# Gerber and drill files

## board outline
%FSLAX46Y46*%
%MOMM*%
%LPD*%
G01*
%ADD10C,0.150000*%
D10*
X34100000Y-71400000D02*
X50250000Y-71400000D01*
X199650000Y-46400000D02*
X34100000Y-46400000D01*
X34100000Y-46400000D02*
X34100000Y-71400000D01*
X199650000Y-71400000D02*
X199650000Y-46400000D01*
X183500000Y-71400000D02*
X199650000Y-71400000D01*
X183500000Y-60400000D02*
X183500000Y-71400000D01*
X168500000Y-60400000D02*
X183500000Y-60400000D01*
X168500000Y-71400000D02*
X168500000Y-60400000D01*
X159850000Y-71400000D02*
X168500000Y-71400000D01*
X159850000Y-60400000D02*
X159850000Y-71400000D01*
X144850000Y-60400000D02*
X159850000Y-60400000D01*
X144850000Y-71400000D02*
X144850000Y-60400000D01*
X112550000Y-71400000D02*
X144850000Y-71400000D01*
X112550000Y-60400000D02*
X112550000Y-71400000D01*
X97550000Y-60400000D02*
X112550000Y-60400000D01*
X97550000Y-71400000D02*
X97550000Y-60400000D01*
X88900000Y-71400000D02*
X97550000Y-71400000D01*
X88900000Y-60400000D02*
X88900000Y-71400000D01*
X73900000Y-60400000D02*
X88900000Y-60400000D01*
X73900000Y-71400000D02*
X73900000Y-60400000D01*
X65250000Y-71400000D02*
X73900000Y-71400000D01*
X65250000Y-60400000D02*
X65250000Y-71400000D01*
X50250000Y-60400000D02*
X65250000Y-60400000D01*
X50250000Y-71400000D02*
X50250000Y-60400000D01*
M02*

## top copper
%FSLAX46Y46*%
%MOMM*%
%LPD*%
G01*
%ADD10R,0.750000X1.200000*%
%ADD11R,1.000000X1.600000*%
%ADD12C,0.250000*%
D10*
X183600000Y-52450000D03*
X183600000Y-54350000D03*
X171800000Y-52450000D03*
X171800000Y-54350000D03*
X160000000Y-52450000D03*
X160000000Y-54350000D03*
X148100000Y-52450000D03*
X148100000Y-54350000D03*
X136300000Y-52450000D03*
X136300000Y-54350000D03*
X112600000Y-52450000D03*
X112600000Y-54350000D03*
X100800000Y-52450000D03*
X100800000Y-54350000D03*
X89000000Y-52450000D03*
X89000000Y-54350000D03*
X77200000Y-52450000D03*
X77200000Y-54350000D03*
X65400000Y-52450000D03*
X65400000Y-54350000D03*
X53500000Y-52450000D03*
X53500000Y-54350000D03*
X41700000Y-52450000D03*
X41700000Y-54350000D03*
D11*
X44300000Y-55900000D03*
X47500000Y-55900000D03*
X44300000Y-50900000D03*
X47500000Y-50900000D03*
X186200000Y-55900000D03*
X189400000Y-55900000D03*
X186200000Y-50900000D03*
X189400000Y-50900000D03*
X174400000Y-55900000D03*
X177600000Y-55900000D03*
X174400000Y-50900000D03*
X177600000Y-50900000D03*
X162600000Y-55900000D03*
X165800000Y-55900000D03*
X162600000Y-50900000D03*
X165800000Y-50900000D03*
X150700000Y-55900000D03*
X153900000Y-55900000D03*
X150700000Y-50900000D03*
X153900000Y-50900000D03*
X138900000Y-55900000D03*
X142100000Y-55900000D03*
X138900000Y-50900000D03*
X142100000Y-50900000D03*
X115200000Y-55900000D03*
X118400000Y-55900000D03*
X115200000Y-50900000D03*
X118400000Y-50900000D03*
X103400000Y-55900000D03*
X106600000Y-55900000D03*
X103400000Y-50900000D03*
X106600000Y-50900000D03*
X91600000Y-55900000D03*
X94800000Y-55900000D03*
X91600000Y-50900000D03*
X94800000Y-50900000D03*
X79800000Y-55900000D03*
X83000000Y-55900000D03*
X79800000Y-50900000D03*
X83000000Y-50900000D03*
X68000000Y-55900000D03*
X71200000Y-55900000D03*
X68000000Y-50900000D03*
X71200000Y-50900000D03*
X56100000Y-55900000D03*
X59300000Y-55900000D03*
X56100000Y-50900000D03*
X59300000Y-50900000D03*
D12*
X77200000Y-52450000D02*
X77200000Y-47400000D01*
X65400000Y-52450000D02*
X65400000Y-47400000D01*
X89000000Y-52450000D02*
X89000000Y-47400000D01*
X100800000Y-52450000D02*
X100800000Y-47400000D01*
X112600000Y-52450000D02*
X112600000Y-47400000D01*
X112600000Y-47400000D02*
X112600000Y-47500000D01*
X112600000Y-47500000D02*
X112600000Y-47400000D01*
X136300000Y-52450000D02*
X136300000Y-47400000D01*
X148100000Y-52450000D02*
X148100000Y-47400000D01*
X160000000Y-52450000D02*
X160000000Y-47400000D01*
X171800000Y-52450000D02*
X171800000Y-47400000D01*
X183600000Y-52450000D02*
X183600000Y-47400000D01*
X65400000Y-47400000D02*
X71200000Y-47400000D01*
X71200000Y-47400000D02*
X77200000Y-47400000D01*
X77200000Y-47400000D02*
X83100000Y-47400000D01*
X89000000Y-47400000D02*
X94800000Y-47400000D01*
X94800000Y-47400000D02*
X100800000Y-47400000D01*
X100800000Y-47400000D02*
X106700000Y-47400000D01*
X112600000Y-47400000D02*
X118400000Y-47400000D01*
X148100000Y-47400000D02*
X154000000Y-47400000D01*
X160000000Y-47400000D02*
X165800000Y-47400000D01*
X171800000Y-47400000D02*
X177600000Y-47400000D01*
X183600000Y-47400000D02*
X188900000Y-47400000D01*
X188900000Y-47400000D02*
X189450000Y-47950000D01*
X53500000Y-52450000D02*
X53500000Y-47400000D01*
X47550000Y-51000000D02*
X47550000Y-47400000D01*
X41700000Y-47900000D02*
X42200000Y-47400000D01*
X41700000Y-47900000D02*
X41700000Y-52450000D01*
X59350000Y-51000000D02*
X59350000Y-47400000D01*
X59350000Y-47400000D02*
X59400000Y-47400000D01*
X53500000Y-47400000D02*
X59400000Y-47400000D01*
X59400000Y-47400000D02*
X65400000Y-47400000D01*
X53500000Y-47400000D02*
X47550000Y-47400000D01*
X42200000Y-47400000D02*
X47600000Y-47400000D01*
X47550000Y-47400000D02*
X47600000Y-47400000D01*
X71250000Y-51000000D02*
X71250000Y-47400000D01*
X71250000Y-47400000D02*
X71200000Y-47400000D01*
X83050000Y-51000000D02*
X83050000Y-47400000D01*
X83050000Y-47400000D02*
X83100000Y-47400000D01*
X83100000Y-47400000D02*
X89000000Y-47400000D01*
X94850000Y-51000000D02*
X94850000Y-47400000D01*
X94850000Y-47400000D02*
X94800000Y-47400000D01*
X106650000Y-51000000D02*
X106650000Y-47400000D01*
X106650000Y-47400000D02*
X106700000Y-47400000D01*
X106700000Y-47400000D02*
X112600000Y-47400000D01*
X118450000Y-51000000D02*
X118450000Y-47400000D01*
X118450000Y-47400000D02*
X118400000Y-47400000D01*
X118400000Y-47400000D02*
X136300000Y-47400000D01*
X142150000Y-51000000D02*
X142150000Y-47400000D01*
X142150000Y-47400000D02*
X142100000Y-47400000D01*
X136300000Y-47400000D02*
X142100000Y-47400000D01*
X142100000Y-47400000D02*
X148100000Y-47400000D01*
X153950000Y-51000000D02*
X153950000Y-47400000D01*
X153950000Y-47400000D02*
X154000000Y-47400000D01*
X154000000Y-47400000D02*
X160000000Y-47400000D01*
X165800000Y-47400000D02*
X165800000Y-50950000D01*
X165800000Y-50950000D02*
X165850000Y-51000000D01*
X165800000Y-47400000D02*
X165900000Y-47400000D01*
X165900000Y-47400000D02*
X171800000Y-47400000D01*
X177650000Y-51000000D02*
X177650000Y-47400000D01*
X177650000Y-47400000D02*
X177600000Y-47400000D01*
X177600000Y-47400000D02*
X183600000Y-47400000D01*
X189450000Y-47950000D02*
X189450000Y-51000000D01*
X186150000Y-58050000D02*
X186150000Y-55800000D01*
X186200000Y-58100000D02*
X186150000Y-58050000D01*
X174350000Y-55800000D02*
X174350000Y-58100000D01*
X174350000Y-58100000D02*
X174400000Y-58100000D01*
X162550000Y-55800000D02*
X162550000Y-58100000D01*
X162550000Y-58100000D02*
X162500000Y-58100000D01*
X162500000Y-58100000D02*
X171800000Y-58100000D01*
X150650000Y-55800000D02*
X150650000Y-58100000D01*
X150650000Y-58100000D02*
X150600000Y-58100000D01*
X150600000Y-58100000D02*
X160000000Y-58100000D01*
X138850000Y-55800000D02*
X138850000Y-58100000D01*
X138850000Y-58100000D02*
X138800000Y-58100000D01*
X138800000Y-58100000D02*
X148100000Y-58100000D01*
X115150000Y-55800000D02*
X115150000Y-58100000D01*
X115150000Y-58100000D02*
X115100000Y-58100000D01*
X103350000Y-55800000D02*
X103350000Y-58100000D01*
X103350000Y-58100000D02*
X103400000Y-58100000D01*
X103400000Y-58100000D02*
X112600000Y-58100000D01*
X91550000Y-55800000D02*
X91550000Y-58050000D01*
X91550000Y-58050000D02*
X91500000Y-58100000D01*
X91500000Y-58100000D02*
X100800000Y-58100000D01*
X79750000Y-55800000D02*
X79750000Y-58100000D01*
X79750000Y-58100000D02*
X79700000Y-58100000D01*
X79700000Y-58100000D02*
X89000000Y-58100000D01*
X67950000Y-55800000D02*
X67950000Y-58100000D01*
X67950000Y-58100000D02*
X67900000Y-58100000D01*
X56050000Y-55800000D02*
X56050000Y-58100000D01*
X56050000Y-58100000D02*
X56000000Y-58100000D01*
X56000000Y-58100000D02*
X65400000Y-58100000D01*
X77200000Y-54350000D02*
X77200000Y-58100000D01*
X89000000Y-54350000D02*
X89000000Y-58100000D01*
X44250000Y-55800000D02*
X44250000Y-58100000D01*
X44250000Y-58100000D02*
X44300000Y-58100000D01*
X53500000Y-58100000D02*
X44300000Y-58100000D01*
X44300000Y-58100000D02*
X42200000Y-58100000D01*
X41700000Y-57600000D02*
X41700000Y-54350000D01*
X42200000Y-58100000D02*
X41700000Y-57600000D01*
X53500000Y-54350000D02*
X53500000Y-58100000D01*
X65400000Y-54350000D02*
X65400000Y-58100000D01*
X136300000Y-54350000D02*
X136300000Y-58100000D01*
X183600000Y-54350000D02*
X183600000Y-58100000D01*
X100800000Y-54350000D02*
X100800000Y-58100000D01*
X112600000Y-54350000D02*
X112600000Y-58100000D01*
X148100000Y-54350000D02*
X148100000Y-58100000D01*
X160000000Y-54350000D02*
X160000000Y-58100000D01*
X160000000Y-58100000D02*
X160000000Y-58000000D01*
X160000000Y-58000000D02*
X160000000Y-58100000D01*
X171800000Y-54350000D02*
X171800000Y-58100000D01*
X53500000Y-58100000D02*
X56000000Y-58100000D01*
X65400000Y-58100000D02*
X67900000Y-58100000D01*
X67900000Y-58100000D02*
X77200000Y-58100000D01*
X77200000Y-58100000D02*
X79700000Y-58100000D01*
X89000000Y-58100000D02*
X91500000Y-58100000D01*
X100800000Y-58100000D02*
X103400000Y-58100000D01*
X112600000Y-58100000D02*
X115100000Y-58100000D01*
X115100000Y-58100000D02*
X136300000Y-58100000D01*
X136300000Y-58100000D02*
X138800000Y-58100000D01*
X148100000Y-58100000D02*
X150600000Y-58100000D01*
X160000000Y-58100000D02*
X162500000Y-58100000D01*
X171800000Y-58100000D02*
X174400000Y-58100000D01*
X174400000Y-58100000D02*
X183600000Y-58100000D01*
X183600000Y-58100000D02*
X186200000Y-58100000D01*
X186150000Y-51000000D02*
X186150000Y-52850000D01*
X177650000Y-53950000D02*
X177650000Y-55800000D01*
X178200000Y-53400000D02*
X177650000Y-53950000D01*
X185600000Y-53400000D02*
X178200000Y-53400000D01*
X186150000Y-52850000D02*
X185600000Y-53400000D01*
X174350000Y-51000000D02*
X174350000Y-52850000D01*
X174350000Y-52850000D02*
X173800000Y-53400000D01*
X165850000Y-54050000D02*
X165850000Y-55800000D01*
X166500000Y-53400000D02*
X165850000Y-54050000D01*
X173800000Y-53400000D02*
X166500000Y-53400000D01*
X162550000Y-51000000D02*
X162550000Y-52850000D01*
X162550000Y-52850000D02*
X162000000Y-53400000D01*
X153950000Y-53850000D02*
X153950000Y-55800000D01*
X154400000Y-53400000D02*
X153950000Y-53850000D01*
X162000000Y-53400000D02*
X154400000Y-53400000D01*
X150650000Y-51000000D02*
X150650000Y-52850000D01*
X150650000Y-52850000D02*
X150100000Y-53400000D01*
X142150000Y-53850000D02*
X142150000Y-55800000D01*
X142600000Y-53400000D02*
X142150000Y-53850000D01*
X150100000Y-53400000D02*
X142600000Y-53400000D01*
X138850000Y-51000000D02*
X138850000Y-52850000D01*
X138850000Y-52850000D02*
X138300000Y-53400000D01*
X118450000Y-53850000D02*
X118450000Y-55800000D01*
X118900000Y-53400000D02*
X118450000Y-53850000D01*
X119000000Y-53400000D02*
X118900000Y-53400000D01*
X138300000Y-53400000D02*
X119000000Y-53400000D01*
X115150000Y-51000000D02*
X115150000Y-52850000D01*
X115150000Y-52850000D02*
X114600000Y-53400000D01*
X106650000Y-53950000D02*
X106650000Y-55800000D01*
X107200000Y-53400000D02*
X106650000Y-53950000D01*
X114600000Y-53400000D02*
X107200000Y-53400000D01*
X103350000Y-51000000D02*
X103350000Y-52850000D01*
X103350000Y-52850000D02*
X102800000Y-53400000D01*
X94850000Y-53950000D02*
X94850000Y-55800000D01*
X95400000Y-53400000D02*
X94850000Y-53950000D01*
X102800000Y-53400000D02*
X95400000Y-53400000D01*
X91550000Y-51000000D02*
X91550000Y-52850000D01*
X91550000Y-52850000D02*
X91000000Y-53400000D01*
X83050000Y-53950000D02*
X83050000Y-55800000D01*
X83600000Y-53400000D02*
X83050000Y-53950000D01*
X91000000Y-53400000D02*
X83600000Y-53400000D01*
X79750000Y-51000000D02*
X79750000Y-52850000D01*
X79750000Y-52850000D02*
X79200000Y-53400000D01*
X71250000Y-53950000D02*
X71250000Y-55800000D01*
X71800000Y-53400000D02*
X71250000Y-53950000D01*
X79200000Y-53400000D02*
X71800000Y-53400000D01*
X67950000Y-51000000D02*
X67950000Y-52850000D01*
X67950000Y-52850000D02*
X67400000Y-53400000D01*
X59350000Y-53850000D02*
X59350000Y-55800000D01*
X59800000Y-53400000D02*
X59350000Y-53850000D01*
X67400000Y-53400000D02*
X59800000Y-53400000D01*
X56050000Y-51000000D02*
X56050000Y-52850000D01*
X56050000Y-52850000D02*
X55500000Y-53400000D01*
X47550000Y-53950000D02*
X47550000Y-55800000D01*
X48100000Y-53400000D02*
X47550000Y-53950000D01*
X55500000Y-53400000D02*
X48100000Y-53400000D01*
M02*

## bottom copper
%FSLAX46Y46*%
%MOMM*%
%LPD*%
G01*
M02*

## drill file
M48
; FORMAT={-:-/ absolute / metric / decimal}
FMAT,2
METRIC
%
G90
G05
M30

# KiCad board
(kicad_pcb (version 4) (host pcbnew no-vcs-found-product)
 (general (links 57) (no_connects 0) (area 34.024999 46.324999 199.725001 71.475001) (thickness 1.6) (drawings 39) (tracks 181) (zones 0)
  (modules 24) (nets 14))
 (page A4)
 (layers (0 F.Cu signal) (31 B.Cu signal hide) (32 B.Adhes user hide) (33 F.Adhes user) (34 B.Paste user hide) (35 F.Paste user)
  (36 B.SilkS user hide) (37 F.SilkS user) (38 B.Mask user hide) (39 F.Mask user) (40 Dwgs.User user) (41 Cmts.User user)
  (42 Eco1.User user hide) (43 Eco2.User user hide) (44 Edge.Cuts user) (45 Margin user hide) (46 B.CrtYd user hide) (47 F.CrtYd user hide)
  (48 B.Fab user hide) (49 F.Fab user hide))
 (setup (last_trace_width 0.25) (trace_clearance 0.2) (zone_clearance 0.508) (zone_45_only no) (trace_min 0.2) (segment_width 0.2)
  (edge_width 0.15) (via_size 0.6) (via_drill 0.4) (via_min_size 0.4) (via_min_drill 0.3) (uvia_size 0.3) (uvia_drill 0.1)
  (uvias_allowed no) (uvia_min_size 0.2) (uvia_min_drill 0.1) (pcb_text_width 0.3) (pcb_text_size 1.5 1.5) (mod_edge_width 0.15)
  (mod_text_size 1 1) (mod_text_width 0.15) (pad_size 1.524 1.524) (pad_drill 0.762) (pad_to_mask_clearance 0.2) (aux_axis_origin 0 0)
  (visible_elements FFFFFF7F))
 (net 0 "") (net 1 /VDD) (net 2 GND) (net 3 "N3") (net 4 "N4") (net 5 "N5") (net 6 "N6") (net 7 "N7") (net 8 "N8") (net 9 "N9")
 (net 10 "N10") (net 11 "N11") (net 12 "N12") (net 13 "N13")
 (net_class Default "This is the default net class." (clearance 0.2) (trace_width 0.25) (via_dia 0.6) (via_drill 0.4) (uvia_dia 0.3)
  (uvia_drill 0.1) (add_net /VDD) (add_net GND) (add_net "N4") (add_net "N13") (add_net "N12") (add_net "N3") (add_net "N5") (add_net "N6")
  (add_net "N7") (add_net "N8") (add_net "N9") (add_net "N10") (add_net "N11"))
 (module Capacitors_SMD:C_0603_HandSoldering (layer F.Cu) (at 183.6 53.4 270)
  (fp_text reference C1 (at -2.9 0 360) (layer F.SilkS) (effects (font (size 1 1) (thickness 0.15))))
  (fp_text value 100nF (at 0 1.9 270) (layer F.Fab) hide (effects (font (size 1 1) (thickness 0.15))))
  (pad 1 smd rect (at -0.95 0 270) (size 1.2 0.75) (layers F.Cu F.Paste F.Mask) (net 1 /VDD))
  (pad 2 smd rect (at 0.95 0 270) (size 1.2 0.75) (layers F.Cu F.Paste F.Mask) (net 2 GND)))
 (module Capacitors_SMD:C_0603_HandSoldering (layer F.Cu) (at 171.8 53.4 270)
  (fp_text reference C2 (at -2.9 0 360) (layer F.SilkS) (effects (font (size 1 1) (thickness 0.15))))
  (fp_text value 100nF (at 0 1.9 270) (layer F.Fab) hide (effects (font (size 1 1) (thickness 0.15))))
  (pad 1 smd rect (at -0.95 0 270) (size 1.2 0.75) (layers F.Cu F.Paste F.Mask) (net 1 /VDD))
  (pad 2 smd rect (at 0.95 0 270) (size 1.2 0.75) (layers F.Cu F.Paste F.Mask) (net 2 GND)))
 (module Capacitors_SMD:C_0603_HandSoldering (layer F.Cu) (at 160 53.4 270)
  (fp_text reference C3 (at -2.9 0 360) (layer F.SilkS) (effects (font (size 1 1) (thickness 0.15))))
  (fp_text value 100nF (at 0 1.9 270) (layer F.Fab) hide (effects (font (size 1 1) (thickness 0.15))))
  (pad 1 smd rect (at -0.95 0 270) (size 1.2 0.75) (layers F.Cu F.Paste F.Mask) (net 1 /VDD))
  (pad 2 smd rect (at 0.95 0 270) (size 1.2 0.75) (layers F.Cu F.Paste F.Mask) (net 2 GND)))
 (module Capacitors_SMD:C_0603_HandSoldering (layer F.Cu) (at 148.1 53.4 270)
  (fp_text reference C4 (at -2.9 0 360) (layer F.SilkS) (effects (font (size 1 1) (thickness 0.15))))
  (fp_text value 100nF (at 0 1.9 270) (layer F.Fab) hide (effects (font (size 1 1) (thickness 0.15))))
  (pad 1 smd rect (at -0.95 0 270) (size 1.2 0.75) (layers F.Cu F.Paste F.Mask) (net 1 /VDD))
  (pad 2 smd rect (at 0.95 0 270) (size 1.2 0.75) (layers F.Cu F.Paste F.Mask) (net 2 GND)))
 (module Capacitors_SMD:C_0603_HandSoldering (layer F.Cu) (at 136.3 53.4 270)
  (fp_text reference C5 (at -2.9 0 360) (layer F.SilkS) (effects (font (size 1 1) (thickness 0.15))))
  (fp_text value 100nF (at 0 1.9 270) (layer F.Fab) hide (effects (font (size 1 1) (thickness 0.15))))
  (pad 1 smd rect (at -0.95 0 270) (size 1.2 0.75) (layers F.Cu F.Paste F.Mask) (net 1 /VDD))
  (pad 2 smd rect (at 0.95 0 270) (size 1.2 0.75) (layers F.Cu F.Paste F.Mask) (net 2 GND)))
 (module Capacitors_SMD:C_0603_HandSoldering (layer F.Cu) (at 112.6 53.4 270)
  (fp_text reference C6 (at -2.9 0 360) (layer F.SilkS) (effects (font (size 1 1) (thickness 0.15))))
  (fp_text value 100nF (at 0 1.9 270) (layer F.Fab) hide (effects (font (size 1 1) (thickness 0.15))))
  (pad 1 smd rect (at -0.95 0 270) (size 1.2 0.75) (layers F.Cu F.Paste F.Mask) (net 1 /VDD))
  (pad 2 smd rect (at 0.95 0 270) (size 1.2 0.75) (layers F.Cu F.Paste F.Mask) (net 2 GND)))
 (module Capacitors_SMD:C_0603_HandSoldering (layer F.Cu) (at 100.8 53.4 270)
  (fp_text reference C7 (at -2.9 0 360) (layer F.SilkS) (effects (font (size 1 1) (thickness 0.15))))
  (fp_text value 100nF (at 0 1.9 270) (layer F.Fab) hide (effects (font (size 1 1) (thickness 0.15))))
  (pad 1 smd rect (at -0.95 0 270) (size 1.2 0.75) (layers F.Cu F.Paste F.Mask) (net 1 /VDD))
  (pad 2 smd rect (at 0.95 0 270) (size 1.2 0.75) (layers F.Cu F.Paste F.Mask) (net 2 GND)))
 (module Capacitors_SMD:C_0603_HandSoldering (layer F.Cu) (at 89 53.4 270)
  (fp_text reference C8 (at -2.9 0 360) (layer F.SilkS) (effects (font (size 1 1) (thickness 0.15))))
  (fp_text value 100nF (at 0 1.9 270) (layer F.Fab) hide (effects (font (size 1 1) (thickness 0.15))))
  (pad 1 smd rect (at -0.95 0 270) (size 1.2 0.75) (layers F.Cu F.Paste F.Mask) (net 1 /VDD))
  (pad 2 smd rect (at 0.95 0 270) (size 1.2 0.75) (layers F.Cu F.Paste F.Mask) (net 2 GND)))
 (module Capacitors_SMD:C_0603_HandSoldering (layer F.Cu) (at 77.2 53.4 270)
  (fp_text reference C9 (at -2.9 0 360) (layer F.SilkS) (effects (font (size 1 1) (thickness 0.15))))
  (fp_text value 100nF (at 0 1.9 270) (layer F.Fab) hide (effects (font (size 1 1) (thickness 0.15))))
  (pad 1 smd rect (at -0.95 0 270) (size 1.2 0.75) (layers F.Cu F.Paste F.Mask) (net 1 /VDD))
  (pad 2 smd rect (at 0.95 0 270) (size 1.2 0.75) (layers F.Cu F.Paste F.Mask) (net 2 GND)))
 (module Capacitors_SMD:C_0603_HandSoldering (layer F.Cu) (at 65.4 53.4 270)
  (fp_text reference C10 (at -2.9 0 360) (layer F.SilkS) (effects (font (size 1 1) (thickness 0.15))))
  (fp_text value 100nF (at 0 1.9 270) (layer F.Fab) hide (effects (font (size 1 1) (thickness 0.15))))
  (pad 1 smd rect (at -0.95 0 270) (size 1.2 0.75) (layers F.Cu F.Paste F.Mask) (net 1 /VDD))
  (pad 2 smd rect (at 0.95 0 270) (size 1.2 0.75) (layers F.Cu F.Paste F.Mask) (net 2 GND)))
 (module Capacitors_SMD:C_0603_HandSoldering (layer F.Cu) (at 53.5 53.4 270)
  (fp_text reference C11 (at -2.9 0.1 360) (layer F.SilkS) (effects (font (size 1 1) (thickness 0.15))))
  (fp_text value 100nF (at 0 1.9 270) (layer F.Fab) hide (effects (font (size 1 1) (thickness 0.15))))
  (pad 1 smd rect (at -0.95 0 270) (size 1.2 0.75) (layers F.Cu F.Paste F.Mask) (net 1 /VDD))
  (pad 2 smd rect (at 0.95 0 270) (size 1.2 0.75) (layers F.Cu F.Paste F.Mask) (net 2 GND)))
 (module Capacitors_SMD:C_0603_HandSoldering (layer F.Cu) (at 41.7 53.4 270)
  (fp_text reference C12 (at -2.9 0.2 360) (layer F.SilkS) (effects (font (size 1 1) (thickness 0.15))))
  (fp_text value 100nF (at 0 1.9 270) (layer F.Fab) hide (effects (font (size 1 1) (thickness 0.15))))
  (pad 1 smd rect (at -0.95 0 270) (size 1.2 0.75) (layers F.Cu F.Paste F.Mask) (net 1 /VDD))
  (pad 2 smd rect (at 0.95 0 270) (size 1.2 0.75) (layers F.Cu F.Paste F.Mask) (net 2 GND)))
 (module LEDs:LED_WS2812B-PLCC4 (layer F.Cu) (at 45.9 53.4 270)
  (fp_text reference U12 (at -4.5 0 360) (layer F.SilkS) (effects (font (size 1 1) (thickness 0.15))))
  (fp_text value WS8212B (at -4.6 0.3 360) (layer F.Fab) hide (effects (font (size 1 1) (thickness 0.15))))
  (pad 3 smd rect (at 2.5 1.6 270) (size 1.6 1) (layers F.Cu F.Paste F.Mask) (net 2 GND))
  (pad 4 smd rect (at 2.5 -1.6 270) (size 1.6 1) (layers F.Cu F.Paste F.Mask) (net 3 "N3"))
  (pad 2 smd rect (at -2.5 1.6 270) (size 1.6 1) (layers F.Cu F.Paste F.Mask))
  (pad 1 smd rect (at -2.5 -1.6 270) (size 1.6 1) (layers F.Cu F.Paste F.Mask) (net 1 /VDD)))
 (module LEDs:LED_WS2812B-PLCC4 (layer F.Cu) (at 187.8 53.4 270)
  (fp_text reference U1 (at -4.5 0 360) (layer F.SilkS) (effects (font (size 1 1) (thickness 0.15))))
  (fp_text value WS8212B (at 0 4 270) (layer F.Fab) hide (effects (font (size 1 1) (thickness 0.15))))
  (pad 3 smd rect (at 2.5 1.6 270) (size 1.6 1) (layers F.Cu F.Paste F.Mask) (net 2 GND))
  (pad 4 smd rect (at 2.5 -1.6 270) (size 1.6 1) (layers F.Cu F.Paste F.Mask))
  (pad 2 smd rect (at -2.5 1.6 270) (size 1.6 1) (layers F.Cu F.Paste F.Mask) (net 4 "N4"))
  (pad 1 smd rect (at -2.5 -1.6 270) (size 1.6 1) (layers F.Cu F.Paste F.Mask) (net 1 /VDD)))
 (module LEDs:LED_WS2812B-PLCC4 (layer F.Cu) (at 176 53.4 270)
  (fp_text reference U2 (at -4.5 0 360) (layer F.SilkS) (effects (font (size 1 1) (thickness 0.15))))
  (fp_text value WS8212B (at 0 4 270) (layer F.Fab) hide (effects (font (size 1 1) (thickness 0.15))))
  (pad 3 smd rect (at 2.5 1.6 270) (size 1.6 1) (layers F.Cu F.Paste F.Mask) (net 2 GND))
  (pad 4 smd rect (at 2.5 -1.6 270) (size 1.6 1) (layers F.Cu F.Paste F.Mask) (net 4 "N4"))
  (pad 2 smd rect (at -2.5 1.6 270) (size 1.6 1) (layers F.Cu F.Paste F.Mask) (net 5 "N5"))
  (pad 1 smd rect (at -2.5 -1.6 270) (size 1.6 1) (layers F.Cu F.Paste F.Mask) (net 1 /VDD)))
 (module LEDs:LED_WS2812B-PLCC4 (layer F.Cu) (at 164.2 53.4 270)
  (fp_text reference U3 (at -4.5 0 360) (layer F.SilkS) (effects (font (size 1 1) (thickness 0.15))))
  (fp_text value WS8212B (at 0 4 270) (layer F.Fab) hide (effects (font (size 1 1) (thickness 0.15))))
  (pad 3 smd rect (at 2.5 1.6 270) (size 1.6 1) (layers F.Cu F.Paste F.Mask) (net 2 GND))
  (pad 4 smd rect (at 2.5 -1.6 270) (size 1.6 1) (layers F.Cu F.Paste F.Mask) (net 5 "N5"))
  (pad 2 smd rect (at -2.5 1.6 270) (size 1.6 1) (layers F.Cu F.Paste F.Mask) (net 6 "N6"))
  (pad 1 smd rect (at -2.5 -1.6 270) (size 1.6 1) (layers F.Cu F.Paste F.Mask) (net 1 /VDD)))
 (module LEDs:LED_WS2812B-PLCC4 (layer F.Cu) (at 152.3 53.4 270)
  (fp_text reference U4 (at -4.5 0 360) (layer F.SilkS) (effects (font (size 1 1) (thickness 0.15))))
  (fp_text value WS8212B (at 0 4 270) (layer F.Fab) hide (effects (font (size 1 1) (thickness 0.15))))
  (pad 3 smd rect (at 2.5 1.6 270) (size 1.6 1) (layers F.Cu F.Paste F.Mask) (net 2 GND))
  (pad 4 smd rect (at 2.5 -1.6 270) (size 1.6 1) (layers F.Cu F.Paste F.Mask) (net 6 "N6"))
  (pad 2 smd rect (at -2.5 1.6 270) (size 1.6 1) (layers F.Cu F.Paste F.Mask) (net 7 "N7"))
  (pad 1 smd rect (at -2.5 -1.6 270) (size 1.6 1) (layers F.Cu F.Paste F.Mask) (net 1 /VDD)))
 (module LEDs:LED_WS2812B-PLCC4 (layer F.Cu) (at 140.5 53.4 270)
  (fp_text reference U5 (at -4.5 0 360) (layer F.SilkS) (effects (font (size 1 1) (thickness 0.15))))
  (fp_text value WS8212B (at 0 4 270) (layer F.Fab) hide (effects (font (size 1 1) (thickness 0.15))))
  (pad 3 smd rect (at 2.5 1.6 270) (size 1.6 1) (layers F.Cu F.Paste F.Mask) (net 2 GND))
  (pad 4 smd rect (at 2.5 -1.6 270) (size 1.6 1) (layers F.Cu F.Paste F.Mask) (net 7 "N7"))
  (pad 2 smd rect (at -2.5 1.6 270) (size 1.6 1) (layers F.Cu F.Paste F.Mask) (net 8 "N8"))
  (pad 1 smd rect (at -2.5 -1.6 270) (size 1.6 1) (layers F.Cu F.Paste F.Mask) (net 1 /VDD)))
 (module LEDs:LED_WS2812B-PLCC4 (layer F.Cu) (at 116.8 53.4 270)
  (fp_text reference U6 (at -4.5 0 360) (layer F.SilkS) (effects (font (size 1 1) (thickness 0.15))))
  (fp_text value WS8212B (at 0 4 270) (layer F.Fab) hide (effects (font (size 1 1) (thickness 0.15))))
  (pad 3 smd rect (at 2.5 1.6 270) (size 1.6 1) (layers F.Cu F.Paste F.Mask) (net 2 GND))
  (pad 4 smd rect (at 2.5 -1.6 270) (size 1.6 1) (layers F.Cu F.Paste F.Mask) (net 8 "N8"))
  (pad 2 smd rect (at -2.5 1.6 270) (size 1.6 1) (layers F.Cu F.Paste F.Mask) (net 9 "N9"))
  (pad 1 smd rect (at -2.5 -1.6 270) (size 1.6 1) (layers F.Cu F.Paste F.Mask) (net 1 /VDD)))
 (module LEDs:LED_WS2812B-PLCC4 (layer F.Cu) (at 105 53.4 270)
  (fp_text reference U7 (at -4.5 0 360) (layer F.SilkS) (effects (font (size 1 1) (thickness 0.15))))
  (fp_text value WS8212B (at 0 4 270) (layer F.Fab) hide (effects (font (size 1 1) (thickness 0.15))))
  (pad 3 smd rect (at 2.5 1.6 270) (size 1.6 1) (layers F.Cu F.Paste F.Mask) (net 2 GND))
  (pad 4 smd rect (at 2.5 -1.6 270) (size 1.6 1) (layers F.Cu F.Paste F.Mask) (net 9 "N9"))
  (pad 2 smd rect (at -2.5 1.6 270) (size 1.6 1) (layers F.Cu F.Paste F.Mask) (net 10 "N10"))
  (pad 1 smd rect (at -2.5 -1.6 270) (size 1.6 1) (layers F.Cu F.Paste F.Mask) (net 1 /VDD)))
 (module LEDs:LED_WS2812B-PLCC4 (layer F.Cu) (at 93.2 53.4 270)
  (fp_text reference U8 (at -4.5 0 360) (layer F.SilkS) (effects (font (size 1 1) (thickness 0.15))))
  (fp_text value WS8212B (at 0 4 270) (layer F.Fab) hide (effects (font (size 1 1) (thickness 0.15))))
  (pad 3 smd rect (at 2.5 1.6 270) (size 1.6 1) (layers F.Cu F.Paste F.Mask) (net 2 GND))
  (pad 4 smd rect (at 2.5 -1.6 270) (size 1.6 1) (layers F.Cu F.Paste F.Mask) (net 10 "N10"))
  (pad 2 smd rect (at -2.5 1.6 270) (size 1.6 1) (layers F.Cu F.Paste F.Mask) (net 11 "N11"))
  (pad 1 smd rect (at -2.5 -1.6 270) (size 1.6 1) (layers F.Cu F.Paste F.Mask) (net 1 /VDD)))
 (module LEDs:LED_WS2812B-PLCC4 (layer F.Cu) (at 81.4 53.4 270)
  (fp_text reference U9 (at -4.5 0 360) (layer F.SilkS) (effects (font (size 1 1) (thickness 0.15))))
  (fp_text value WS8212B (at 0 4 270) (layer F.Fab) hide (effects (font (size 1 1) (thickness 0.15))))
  (pad 3 smd rect (at 2.5 1.6 270) (size 1.6 1) (layers F.Cu F.Paste F.Mask) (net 2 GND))
  (pad 4 smd rect (at 2.5 -1.6 270) (size 1.6 1) (layers F.Cu F.Paste F.Mask) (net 11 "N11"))
  (pad 2 smd rect (at -2.5 1.6 270) (size 1.6 1) (layers F.Cu F.Paste F.Mask) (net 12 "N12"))
  (pad 1 smd rect (at -2.5 -1.6 270) (size 1.6 1) (layers F.Cu F.Paste F.Mask) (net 1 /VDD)))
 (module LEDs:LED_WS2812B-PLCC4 (layer F.Cu) (at 69.6 53.4 270)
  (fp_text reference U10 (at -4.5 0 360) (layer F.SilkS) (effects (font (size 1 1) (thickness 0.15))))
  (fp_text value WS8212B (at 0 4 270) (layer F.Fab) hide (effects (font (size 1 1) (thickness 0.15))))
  (pad 3 smd rect (at 2.5 1.6 270) (size 1.6 1) (layers F.Cu F.Paste F.Mask) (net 2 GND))
  (pad 4 smd rect (at 2.5 -1.6 270) (size 1.6 1) (layers F.Cu F.Paste F.Mask) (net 12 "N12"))
  (pad 2 smd rect (at -2.5 1.6 270) (size 1.6 1) (layers F.Cu F.Paste F.Mask) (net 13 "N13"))
  (pad 1 smd rect (at -2.5 -1.6 270) (size 1.6 1) (layers F.Cu F.Paste F.Mask) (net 1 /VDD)))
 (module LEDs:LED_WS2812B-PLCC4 (layer F.Cu) (at 57.7 53.4 270)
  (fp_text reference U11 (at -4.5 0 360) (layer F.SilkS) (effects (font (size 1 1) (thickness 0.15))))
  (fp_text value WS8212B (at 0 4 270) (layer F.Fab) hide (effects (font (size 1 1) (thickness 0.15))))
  (pad 3 smd rect (at 2.5 1.6 270) (size 1.6 1) (layers F.Cu F.Paste F.Mask) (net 2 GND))
  (pad 4 smd rect (at 2.5 -1.6 270) (size 1.6 1) (layers F.Cu F.Paste F.Mask) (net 13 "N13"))
  (pad 2 smd rect (at -2.5 1.6 270) (size 1.6 1) (layers F.Cu F.Paste F.Mask) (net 3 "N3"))
  (pad 1 smd rect (at -2.5 -1.6 270) (size 1.6 1) (layers F.Cu F.Paste F.Mask) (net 1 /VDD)))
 (gr_line (start 34.1 71.4) (end 50.25 71.4) (angle 90) (layer Edge.Cuts) (width 0.15))
 (gr_line (start 199.65 46.4) (end 34.1 46.4) (angle 90) (layer Edge.Cuts) (width 0.15))
 (gr_line (start 34.1 46.4) (end 34.1 71.4) (angle 90) (layer Edge.Cuts) (width 0.15))
 (gr_line (start 199.65 71.4) (end 199.65 46.4) (angle 90) (layer Edge.Cuts) (width 0.15))
 (gr_line (start 183.5 71.4) (end 199.65 71.4) (angle 90) (layer Edge.Cuts) (width 0.15))
 (gr_line (start 183.5 60.4) (end 183.5 71.4) (angle 90) (layer Edge.Cuts) (width 0.15))
 (gr_line (start 168.5 60.4) (end 183.5 60.4) (angle 90) (layer Edge.Cuts) (width 0.15))
 (gr_line (start 168.5 71.4) (end 168.5 60.4) (angle 90) (layer Edge.Cuts) (width 0.15))
 (gr_line (start 159.85 71.4) (end 168.5 71.4) (angle 90) (layer Edge.Cuts) (width 0.15))
 (gr_line (start 159.85 60.4) (end 159.85 71.4) (angle 90) (layer Edge.Cuts) (width 0.15))
 (gr_line (start 144.85 60.4) (end 159.85 60.4) (angle 90) (layer Edge.Cuts) (width 0.15))
 (gr_line (start 144.85 71.4) (end 144.85 60.4) (angle 90) (layer Edge.Cuts) (width 0.15))
 (gr_line (start 112.55 71.4) (end 144.85 71.4) (angle 90) (layer Edge.Cuts) (width 0.15))
 (gr_line (start 112.55 60.4) (end 112.55 71.4) (angle 90) (layer Edge.Cuts) (width 0.15))
 (gr_line (start 97.55 60.4) (end 112.55 60.4) (angle 90) (layer Edge.Cuts) (width 0.15))
 (gr_line (start 97.55 71.4) (end 97.55 60.4) (angle 90) (layer Edge.Cuts) (width 0.15))
 (gr_line (start 88.9 71.4) (end 97.55 71.4) (angle 90) (layer Edge.Cuts) (width 0.15))
 (gr_line (start 88.9 60.4) (end 88.9 71.4) (angle 90) (layer Edge.Cuts) (width 0.15))
 (gr_line (start 73.9 60.4) (end 88.9 60.4) (angle 90) (layer Edge.Cuts) (width 0.15))
 (gr_line (start 73.9 71.4) (end 73.9 60.4) (angle 90) (layer Edge.Cuts) (width 0.15))
 (gr_line (start 65.25 71.4) (end 73.9 71.4) (angle 90) (layer Edge.Cuts) (width 0.15))
 (gr_line (start 65.25 60.4) (end 65.25 71.4) (angle 90) (layer Edge.Cuts) (width 0.15))
 (gr_line (start 50.25 60.4) (end 65.25 60.4) (angle 90) (layer Edge.Cuts) (width 0.15))
 (gr_line (start 50.25 71.4) (end 50.25 60.4) (angle 90) (layer Edge.Cuts) (width 0.15))
 (segment (start 77.2 52.45) (end 77.2 47.4) (width 0.25) (layer F.Cu) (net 1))
 (segment (start 65.4 52.45) (end 65.4 47.4) (width 0.25) (layer F.Cu) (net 1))
 (segment (start 89 52.45) (end 89 47.4) (width 0.25) (layer F.Cu) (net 1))
 (segment (start 100.8 52.45) (end 100.8 47.4) (width 0.25) (layer F.Cu) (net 1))
 (segment (start 112.6 52.45) (end 112.6 47.4) (width 0.25) (layer F.Cu) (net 1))
 (segment (start 112.6 47.4) (end 112.6 47.5) (width 0.25) (layer F.Cu) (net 1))
 (segment (start 112.6 47.5) (end 112.6 47.4) (width 0.25) (layer F.Cu) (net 1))
 (segment (start 136.3 52.45) (end 136.3 47.4) (width 0.25) (layer F.Cu) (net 1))
 (segment (start 148.1 52.45) (end 148.1 47.4) (width 0.25) (layer F.Cu) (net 1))
 (segment (start 160 52.45) (end 160 47.4) (width 0.25) (layer F.Cu) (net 1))
 (segment (start 171.8 52.45) (end 171.8 47.4) (width 0.25) (layer F.Cu) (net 1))
 (segment (start 183.6 52.45) (end 183.6 47.4) (width 0.25) (layer F.Cu) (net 1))
 (segment (start 65.4 47.4) (end 71.2 47.4) (width 0.25) (layer F.Cu) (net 1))
 (segment (start 71.2 47.4) (end 77.2 47.4) (width 0.25) (layer F.Cu) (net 1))
 (segment (start 77.2 47.4) (end 83.1 47.4) (width 0.25) (layer F.Cu) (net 1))
 (segment (start 89 47.4) (end 94.8 47.4) (width 0.25) (layer F.Cu) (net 1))
 (segment (start 94.8 47.4) (end 100.8 47.4) (width 0.25) (layer F.Cu) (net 1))
 (segment (start 100.8 47.4) (end 106.7 47.4) (width 0.25) (layer F.Cu) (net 1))
 (segment (start 112.6 47.4) (end 118.4 47.4) (width 0.25) (layer F.Cu) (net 1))
 (segment (start 148.1 47.4) (end 154 47.4) (width 0.25) (layer F.Cu) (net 1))
 (segment (start 160 47.4) (end 165.8 47.4) (width 0.25) (layer F.Cu) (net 1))
 (segment (start 171.8 47.4) (end 177.6 47.4) (width 0.25) (layer F.Cu) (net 1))
 (segment (start 183.6 47.4) (end 188.9 47.4) (width 0.25) (layer F.Cu) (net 1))
 (segment (start 188.9 47.4) (end 189.45 47.95) (width 0.25) (layer F.Cu) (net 1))
 (segment (start 53.5 52.45) (end 53.5 47.4) (width 0.25) (layer F.Cu) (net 1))
 (segment (start 47.55 51) (end 47.55 47.4) (width 0.25) (layer F.Cu) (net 1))
 (segment (start 41.7 47.9) (end 42.2 47.4) (width 0.25) (layer F.Cu) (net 1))
 (segment (start 41.7 47.9) (end 41.7 52.45) (width 0.25) (layer F.Cu) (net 1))
 (segment (start 59.35 51) (end 59.35 47.4) (width 0.25) (layer F.Cu) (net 1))
 (segment (start 59.35 47.4) (end 59.4 47.4) (width 0.25) (layer F.Cu) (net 1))
 (segment (start 53.5 47.4) (end 59.4 47.4) (width 0.25) (layer F.Cu) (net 1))
 (segment (start 59.4 47.4) (end 65.4 47.4) (width 0.25) (layer F.Cu) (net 1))
 (segment (start 53.5 47.4) (end 47.55 47.4) (width 0.25) (layer F.Cu) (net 1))
 (segment (start 42.2 47.4) (end 47.6 47.4) (width 0.25) (layer F.Cu) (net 1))
 (segment (start 47.55 47.4) (end 47.6 47.4) (width 0.25) (layer F.Cu) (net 1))
 (segment (start 71.25 51) (end 71.25 47.4) (width 0.25) (layer F.Cu) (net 1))
 (segment (start 71.25 47.4) (end 71.2 47.4) (width 0.25) (layer F.Cu) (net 1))
 (segment (start 83.05 51) (end 83.05 47.4) (width 0.25) (layer F.Cu) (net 1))
 (segment (start 83.05 47.4) (end 83.1 47.4) (width 0.25) (layer F.Cu) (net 1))
 (segment (start 83.1 47.4) (end 89 47.4) (width 0.25) (layer F.Cu) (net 1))
 (segment (start 94.85 51) (end 94.85 47.4) (width 0.25) (layer F.Cu) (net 1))
 (segment (start 94.85 47.4) (end 94.8 47.4) (width 0.25) (layer F.Cu) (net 1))
 (segment (start 106.65 51) (end 106.65 47.4) (width 0.25) (layer F.Cu) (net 1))
 (segment (start 106.65 47.4) (end 106.7 47.4) (width 0.25) (layer F.Cu) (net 1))
 (segment (start 106.7 47.4) (end 112.6 47.4) (width 0.25) (layer F.Cu) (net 1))
 (segment (start 118.45 51) (end 118.45 47.4) (width 0.25) (layer F.Cu) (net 1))
 (segment (start 118.45 47.4) (end 118.4 47.4) (width 0.25) (layer F.Cu) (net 1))
 (segment (start 118.4 47.4) (end 136.3 47.4) (width 0.25) (layer F.Cu) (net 1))
 (segment (start 142.15 51) (end 142.15 47.4) (width 0.25) (layer F.Cu) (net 1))
 (segment (start 142.15 47.4) (end 142.1 47.4) (width 0.25) (layer F.Cu) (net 1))
 (segment (start 136.3 47.4) (end 142.1 47.4) (width 0.25) (layer F.Cu) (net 1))
 (segment (start 142.1 47.4) (end 148.1 47.4) (width 0.25) (layer F.Cu) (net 1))
 (segment (start 153.95 51) (end 153.95 47.4) (width 0.25) (layer F.Cu) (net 1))
 (segment (start 153.95 47.4) (end 154 47.4) (width 0.25) (layer F.Cu) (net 1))
 (segment (start 154 47.4) (end 160 47.4) (width 0.25) (layer F.Cu) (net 1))
 (segment (start 165.8 47.4) (end 165.8 50.95) (width 0.25) (layer F.Cu) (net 1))
 (segment (start 165.8 50.95) (end 165.85 51) (width 0.25) (layer F.Cu) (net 1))
 (segment (start 165.8 47.4) (end 165.9 47.4) (width 0.25) (layer F.Cu) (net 1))
 (segment (start 165.9 47.4) (end 171.8 47.4) (width 0.25) (layer F.Cu) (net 1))
 (segment (start 177.65 51) (end 177.65 47.4) (width 0.25) (layer F.Cu) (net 1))
 (segment (start 177.65 47.4) (end 177.6 47.4) (width 0.25) (layer F.Cu) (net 1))
 (segment (start 177.6 47.4) (end 183.6 47.4) (width 0.25) (layer F.Cu) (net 1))
 (segment (start 189.45 47.95) (end 189.45 51) (width 0.25) (layer F.Cu) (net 1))
 (segment (start 186.15 58.05) (end 186.15 55.8) (width 0.25) (layer F.Cu) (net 2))
 (segment (start 186.2 58.1) (end 186.15 58.05) (width 0.25) (layer F.Cu) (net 2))
 (segment (start 174.35 55.8) (end 174.35 58.1) (width 0.25) (layer F.Cu) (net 2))
 (segment (start 174.35 58.1) (end 174.4 58.1) (width 0.25) (layer F.Cu) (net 2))
 (segment (start 162.55 55.8) (end 162.55 58.1) (width 0.25) (layer F.Cu) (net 2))
 (segment (start 162.55 58.1) (end 162.5 58.1) (width 0.25) (layer F.Cu) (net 2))
 (segment (start 162.5 58.1) (end 171.8 58.1) (width 0.25) (layer F.Cu) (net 2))
 (segment (start 150.65 55.8) (end 150.65 58.1) (width 0.25) (layer F.Cu) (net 2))
 (segment (start 150.65 58.1) (end 150.6 58.1) (width 0.25) (layer F.Cu) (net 2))
 (segment (start 150.6 58.1) (end 160 58.1) (width 0.25) (layer F.Cu) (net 2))
 (segment (start 138.85 55.8) (end 138.85 58.1) (width 0.25) (layer F.Cu) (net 2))
 (segment (start 138.85 58.1) (end 138.8 58.1) (width 0.25) (layer F.Cu) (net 2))
 (segment (start 138.8 58.1) (end 148.1 58.1) (width 0.25) (layer F.Cu) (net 2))
 (segment (start 115.15 55.8) (end 115.15 58.1) (width 0.25) (layer F.Cu) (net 2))
 (segment (start 115.15 58.1) (end 115.1 58.1) (width 0.25) (layer F.Cu) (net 2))
 (segment (start 103.35 55.8) (end 103.35 58.1) (width 0.25) (layer F.Cu) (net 2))
 (segment (start 103.35 58.1) (end 103.4 58.1) (width 0.25) (layer F.Cu) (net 2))
 (segment (start 103.4 58.1) (end 112.6 58.1) (width 0.25) (layer F.Cu) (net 2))
 (segment (start 91.55 55.8) (end 91.55 58.05) (width 0.25) (layer F.Cu) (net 2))
 (segment (start 91.55 58.05) (end 91.5 58.1) (width 0.25) (layer F.Cu) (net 2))
 (segment (start 91.5 58.1) (end 100.8 58.1) (width 0.25) (layer F.Cu) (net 2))
 (segment (start 79.75 55.8) (end 79.75 58.1) (width 0.25) (layer F.Cu) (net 2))
 (segment (start 79.75 58.1) (end 79.7 58.1) (width 0.25) (layer F.Cu) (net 2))
 (segment (start 79.7 58.1) (end 89 58.1) (width 0.25) (layer F.Cu) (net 2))
 (segment (start 67.95 55.8) (end 67.95 58.1) (width 0.25) (layer F.Cu) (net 2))
 (segment (start 67.95 58.1) (end 67.9 58.1) (width 0.25) (layer F.Cu) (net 2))
 (segment (start 56.05 55.8) (end 56.05 58.1) (width 0.25) (layer F.Cu) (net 2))
 (segment (start 56.05 58.1) (end 56 58.1) (width 0.25) (layer F.Cu) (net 2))
 (segment (start 56 58.1) (end 65.4 58.1) (width 0.25) (layer F.Cu) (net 2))
 (segment (start 77.2 54.35) (end 77.2 58.1) (width 0.25) (layer F.Cu) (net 2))
 (segment (start 89 54.35) (end 89 58.1) (width 0.25) (layer F.Cu) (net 2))
 (segment (start 44.25 55.8) (end 44.25 58.1) (width 0.25) (layer F.Cu) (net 2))
 (segment (start 44.25 58.1) (end 44.3 58.1) (width 0.25) (layer F.Cu) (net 2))
 (segment (start 53.5 58.1) (end 44.3 58.1) (width 0.25) (layer F.Cu) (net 2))
 (segment (start 44.3 58.1) (end 42.2 58.1) (width 0.25) (layer F.Cu) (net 2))
 (segment (start 41.7 57.6) (end 41.7 54.35) (width 0.25) (layer F.Cu) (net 2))
 (segment (start 42.2 58.1) (end 41.7 57.6) (width 0.25) (layer F.Cu) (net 2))
 (segment (start 53.5 54.35) (end 53.5 58.1) (width 0.25) (layer F.Cu) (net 2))
 (segment (start 65.4 54.35) (end 65.4 58.1) (width 0.25) (layer F.Cu) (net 2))
 (segment (start 136.3 54.35) (end 136.3 58.1) (width 0.25) (layer F.Cu) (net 2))
 (segment (start 183.6 54.35) (end 183.6 58.1) (width 0.25) (layer F.Cu) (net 2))
 (segment (start 100.8 54.35) (end 100.8 58.1) (width 0.25) (layer F.Cu) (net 2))
 (segment (start 112.6 54.35) (end 112.6 58.1) (width 0.25) (layer F.Cu) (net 2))
 (segment (start 148.1 54.35) (end 148.1 58.1) (width 0.25) (layer F.Cu) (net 2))
 (segment (start 160 54.35) (end 160 58.1) (width 0.25) (layer F.Cu) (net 2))
 (segment (start 160 58.1) (end 160 58) (width 0.25) (layer F.Cu) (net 2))
 (segment (start 160 58) (end 160 58.1) (width 0.25) (layer F.Cu) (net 2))
 (segment (start 171.8 54.35) (end 171.8 58.1) (width 0.25) (layer F.Cu) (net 2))
 (segment (start 53.5 58.1) (end 56 58.1) (width 0.25) (layer F.Cu) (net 2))
 (segment (start 65.4 58.1) (end 67.9 58.1) (width 0.25) (layer F.Cu) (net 2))
 (segment (start 67.9 58.1) (end 77.2 58.1) (width 0.25) (layer F.Cu) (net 2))
 (segment (start 77.2 58.1) (end 79.7 58.1) (width 0.25) (layer F.Cu) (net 2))
 (segment (start 89 58.1) (end 91.5 58.1) (width 0.25) (layer F.Cu) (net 2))
 (segment (start 100.8 58.1) (end 103.4 58.1) (width 0.25) (layer F.Cu) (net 2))
 (segment (start 112.6 58.1) (end 115.1 58.1) (width 0.25) (layer F.Cu) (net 2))
 (segment (start 115.1 58.1) (end 136.3 58.1) (width 0.25) (layer F.Cu) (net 2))
 (segment (start 136.3 58.1) (end 138.8 58.1) (width 0.25) (layer F.Cu) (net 2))
 (segment (start 148.1 58.1) (end 150.6 58.1) (width 0.25) (layer F.Cu) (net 2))
 (segment (start 160 58.1) (end 162.5 58.1) (width 0.25) (layer F.Cu) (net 2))
 (segment (start 171.8 58.1) (end 174.4 58.1) (width 0.25) (layer F.Cu) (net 2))
 (segment (start 174.4 58.1) (end 183.6 58.1) (width 0.25) (layer F.Cu) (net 2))
 (segment (start 183.6 58.1) (end 186.2 58.1) (width 0.25) (layer F.Cu) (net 2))
 (segment (start 186.15 51) (end 186.15 52.85) (width 0.25) (layer F.Cu) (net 4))
 (segment (start 177.65 53.95) (end 177.65 55.8) (width 0.25) (layer F.Cu) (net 4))
 (segment (start 178.2 53.4) (end 177.65 53.95) (width 0.25) (layer F.Cu) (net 4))
 (segment (start 185.6 53.4) (end 178.2 53.4) (width 0.25) (layer F.Cu) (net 4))
 (segment (start 186.15 52.85) (end 185.6 53.4) (width 0.25) (layer F.Cu) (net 4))
 (segment (start 174.35 51) (end 174.35 52.85) (width 0.25) (layer F.Cu) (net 5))
 (segment (start 174.35 52.85) (end 173.8 53.4) (width 0.25) (layer F.Cu) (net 5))
 (segment (start 165.85 54.05) (end 165.85 55.8) (width 0.25) (layer F.Cu) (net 5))
 (segment (start 166.5 53.4) (end 165.85 54.05) (width 0.25) (layer F.Cu) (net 5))
 (segment (start 173.8 53.4) (end 166.5 53.4) (width 0.25) (layer F.Cu) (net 5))
 (segment (start 162.55 51) (end 162.55 52.85) (width 0.25) (layer F.Cu) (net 6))
 (segment (start 162.55 52.85) (end 162 53.4) (width 0.25) (layer F.Cu) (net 6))
 (segment (start 153.95 53.85) (end 153.95 55.8) (width 0.25) (layer F.Cu) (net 6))
 (segment (start 154.4 53.4) (end 153.95 53.85) (width 0.25) (layer F.Cu) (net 6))
 (segment (start 162 53.4) (end 154.4 53.4) (width 0.25) (layer F.Cu) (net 6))
 (segment (start 150.65 51) (end 150.65 52.85) (width 0.25) (layer F.Cu) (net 7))
 (segment (start 150.65 52.85) (end 150.1 53.4) (width 0.25) (layer F.Cu) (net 7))
 (segment (start 142.15 53.85) (end 142.15 55.8) (width 0.25) (layer F.Cu) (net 7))
 (segment (start 142.6 53.4) (end 142.15 53.85) (width 0.25) (layer F.Cu) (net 7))
 (segment (start 150.1 53.4) (end 142.6 53.4) (width 0.25) (layer F.Cu) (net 7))
 (segment (start 138.85 51) (end 138.85 52.85) (width 0.25) (layer F.Cu) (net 8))
 (segment (start 138.85 52.85) (end 138.3 53.4) (width 0.25) (layer F.Cu) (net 8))
 (segment (start 118.45 53.85) (end 118.45 55.8) (width 0.25) (layer F.Cu) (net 8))
 (segment (start 118.9 53.4) (end 118.45 53.85) (width 0.25) (layer F.Cu) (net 8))
 (segment (start 119 53.4) (end 118.9 53.4) (width 0.25) (layer F.Cu) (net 8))
 (segment (start 138.3 53.4) (end 119 53.4) (width 0.25) (layer F.Cu) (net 8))
 (segment (start 115.15 51) (end 115.15 52.85) (width 0.25) (layer F.Cu) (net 9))
 (segment (start 115.15 52.85) (end 114.6 53.4) (width 0.25) (layer F.Cu) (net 9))
 (segment (start 106.65 53.95) (end 106.65 55.8) (width 0.25) (layer F.Cu) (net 9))
 (segment (start 107.2 53.4) (end 106.65 53.95) (width 0.25) (layer F.Cu) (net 9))
 (segment (start 114.6 53.4) (end 107.2 53.4) (width 0.25) (layer F.Cu) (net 9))
 (segment (start 103.35 51) (end 103.35 52.85) (width 0.25) (layer F.Cu) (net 10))
 (segment (start 103.35 52.85) (end 102.8 53.4) (width 0.25) (layer F.Cu) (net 10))
 (segment (start 94.85 53.95) (end 94.85 55.8) (width 0.25) (layer F.Cu) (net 10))
 (segment (start 95.4 53.4) (end 94.85 53.95) (width 0.25) (layer F.Cu) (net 10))
 (segment (start 102.8 53.4) (end 95.4 53.4) (width 0.25) (layer F.Cu) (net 10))
 (segment (start 91.55 51) (end 91.55 52.85) (width 0.25) (layer F.Cu) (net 11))
 (segment (start 91.55 52.85) (end 91 53.4) (width 0.25) (layer F.Cu) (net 11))
 (segment (start 83.05 53.95) (end 83.05 55.8) (width 0.25) (layer F.Cu) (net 11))
 (segment (start 83.6 53.4) (end 83.05 53.95) (width 0.25) (layer F.Cu) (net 11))
 (segment (start 91 53.4) (end 83.6 53.4) (width 0.25) (layer F.Cu) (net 11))
 (segment (start 79.75 51) (end 79.75 52.85) (width 0.25) (layer F.Cu) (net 12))
 (segment (start 79.75 52.85) (end 79.2 53.4) (width 0.25) (layer F.Cu) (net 12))
 (segment (start 71.25 53.95) (end 71.25 55.8) (width 0.25) (layer F.Cu) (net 12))
 (segment (start 71.8 53.4) (end 71.25 53.95) (width 0.25) (layer F.Cu) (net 12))
 (segment (start 79.2 53.4) (end 71.8 53.4) (width 0.25) (layer F.Cu) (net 12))
 (segment (start 67.95 51) (end 67.95 52.85) (width 0.25) (layer F.Cu) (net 13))
 (segment (start 67.95 52.85) (end 67.4 53.4) (width 0.25) (layer F.Cu) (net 13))
 (segment (start 59.35 53.85) (end 59.35 55.8) (width 0.25) (layer F.Cu) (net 13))
 (segment (start 59.8 53.4) (end 59.35 53.85) (width 0.25) (layer F.Cu) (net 13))
 (segment (start 67.4 53.4) (end 59.8 53.4) (width 0.25) (layer F.Cu) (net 13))
 (segment (start 56.05 51) (end 56.05 52.85) (width 0.25) (layer F.Cu) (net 3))
 (segment (start 56.05 52.85) (end 55.5 53.4) (width 0.25) (layer F.Cu) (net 3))
 (segment (start 47.55 53.95) (end 47.55 55.8) (width 0.25) (layer F.Cu) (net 3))
 (segment (start 48.1 53.4) (end 47.55 53.95) (width 0.25) (layer F.Cu) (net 3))
 (segment (start 55.5 53.4) (end 48.1 53.4) (width 0.25) (layer F.Cu) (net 3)))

